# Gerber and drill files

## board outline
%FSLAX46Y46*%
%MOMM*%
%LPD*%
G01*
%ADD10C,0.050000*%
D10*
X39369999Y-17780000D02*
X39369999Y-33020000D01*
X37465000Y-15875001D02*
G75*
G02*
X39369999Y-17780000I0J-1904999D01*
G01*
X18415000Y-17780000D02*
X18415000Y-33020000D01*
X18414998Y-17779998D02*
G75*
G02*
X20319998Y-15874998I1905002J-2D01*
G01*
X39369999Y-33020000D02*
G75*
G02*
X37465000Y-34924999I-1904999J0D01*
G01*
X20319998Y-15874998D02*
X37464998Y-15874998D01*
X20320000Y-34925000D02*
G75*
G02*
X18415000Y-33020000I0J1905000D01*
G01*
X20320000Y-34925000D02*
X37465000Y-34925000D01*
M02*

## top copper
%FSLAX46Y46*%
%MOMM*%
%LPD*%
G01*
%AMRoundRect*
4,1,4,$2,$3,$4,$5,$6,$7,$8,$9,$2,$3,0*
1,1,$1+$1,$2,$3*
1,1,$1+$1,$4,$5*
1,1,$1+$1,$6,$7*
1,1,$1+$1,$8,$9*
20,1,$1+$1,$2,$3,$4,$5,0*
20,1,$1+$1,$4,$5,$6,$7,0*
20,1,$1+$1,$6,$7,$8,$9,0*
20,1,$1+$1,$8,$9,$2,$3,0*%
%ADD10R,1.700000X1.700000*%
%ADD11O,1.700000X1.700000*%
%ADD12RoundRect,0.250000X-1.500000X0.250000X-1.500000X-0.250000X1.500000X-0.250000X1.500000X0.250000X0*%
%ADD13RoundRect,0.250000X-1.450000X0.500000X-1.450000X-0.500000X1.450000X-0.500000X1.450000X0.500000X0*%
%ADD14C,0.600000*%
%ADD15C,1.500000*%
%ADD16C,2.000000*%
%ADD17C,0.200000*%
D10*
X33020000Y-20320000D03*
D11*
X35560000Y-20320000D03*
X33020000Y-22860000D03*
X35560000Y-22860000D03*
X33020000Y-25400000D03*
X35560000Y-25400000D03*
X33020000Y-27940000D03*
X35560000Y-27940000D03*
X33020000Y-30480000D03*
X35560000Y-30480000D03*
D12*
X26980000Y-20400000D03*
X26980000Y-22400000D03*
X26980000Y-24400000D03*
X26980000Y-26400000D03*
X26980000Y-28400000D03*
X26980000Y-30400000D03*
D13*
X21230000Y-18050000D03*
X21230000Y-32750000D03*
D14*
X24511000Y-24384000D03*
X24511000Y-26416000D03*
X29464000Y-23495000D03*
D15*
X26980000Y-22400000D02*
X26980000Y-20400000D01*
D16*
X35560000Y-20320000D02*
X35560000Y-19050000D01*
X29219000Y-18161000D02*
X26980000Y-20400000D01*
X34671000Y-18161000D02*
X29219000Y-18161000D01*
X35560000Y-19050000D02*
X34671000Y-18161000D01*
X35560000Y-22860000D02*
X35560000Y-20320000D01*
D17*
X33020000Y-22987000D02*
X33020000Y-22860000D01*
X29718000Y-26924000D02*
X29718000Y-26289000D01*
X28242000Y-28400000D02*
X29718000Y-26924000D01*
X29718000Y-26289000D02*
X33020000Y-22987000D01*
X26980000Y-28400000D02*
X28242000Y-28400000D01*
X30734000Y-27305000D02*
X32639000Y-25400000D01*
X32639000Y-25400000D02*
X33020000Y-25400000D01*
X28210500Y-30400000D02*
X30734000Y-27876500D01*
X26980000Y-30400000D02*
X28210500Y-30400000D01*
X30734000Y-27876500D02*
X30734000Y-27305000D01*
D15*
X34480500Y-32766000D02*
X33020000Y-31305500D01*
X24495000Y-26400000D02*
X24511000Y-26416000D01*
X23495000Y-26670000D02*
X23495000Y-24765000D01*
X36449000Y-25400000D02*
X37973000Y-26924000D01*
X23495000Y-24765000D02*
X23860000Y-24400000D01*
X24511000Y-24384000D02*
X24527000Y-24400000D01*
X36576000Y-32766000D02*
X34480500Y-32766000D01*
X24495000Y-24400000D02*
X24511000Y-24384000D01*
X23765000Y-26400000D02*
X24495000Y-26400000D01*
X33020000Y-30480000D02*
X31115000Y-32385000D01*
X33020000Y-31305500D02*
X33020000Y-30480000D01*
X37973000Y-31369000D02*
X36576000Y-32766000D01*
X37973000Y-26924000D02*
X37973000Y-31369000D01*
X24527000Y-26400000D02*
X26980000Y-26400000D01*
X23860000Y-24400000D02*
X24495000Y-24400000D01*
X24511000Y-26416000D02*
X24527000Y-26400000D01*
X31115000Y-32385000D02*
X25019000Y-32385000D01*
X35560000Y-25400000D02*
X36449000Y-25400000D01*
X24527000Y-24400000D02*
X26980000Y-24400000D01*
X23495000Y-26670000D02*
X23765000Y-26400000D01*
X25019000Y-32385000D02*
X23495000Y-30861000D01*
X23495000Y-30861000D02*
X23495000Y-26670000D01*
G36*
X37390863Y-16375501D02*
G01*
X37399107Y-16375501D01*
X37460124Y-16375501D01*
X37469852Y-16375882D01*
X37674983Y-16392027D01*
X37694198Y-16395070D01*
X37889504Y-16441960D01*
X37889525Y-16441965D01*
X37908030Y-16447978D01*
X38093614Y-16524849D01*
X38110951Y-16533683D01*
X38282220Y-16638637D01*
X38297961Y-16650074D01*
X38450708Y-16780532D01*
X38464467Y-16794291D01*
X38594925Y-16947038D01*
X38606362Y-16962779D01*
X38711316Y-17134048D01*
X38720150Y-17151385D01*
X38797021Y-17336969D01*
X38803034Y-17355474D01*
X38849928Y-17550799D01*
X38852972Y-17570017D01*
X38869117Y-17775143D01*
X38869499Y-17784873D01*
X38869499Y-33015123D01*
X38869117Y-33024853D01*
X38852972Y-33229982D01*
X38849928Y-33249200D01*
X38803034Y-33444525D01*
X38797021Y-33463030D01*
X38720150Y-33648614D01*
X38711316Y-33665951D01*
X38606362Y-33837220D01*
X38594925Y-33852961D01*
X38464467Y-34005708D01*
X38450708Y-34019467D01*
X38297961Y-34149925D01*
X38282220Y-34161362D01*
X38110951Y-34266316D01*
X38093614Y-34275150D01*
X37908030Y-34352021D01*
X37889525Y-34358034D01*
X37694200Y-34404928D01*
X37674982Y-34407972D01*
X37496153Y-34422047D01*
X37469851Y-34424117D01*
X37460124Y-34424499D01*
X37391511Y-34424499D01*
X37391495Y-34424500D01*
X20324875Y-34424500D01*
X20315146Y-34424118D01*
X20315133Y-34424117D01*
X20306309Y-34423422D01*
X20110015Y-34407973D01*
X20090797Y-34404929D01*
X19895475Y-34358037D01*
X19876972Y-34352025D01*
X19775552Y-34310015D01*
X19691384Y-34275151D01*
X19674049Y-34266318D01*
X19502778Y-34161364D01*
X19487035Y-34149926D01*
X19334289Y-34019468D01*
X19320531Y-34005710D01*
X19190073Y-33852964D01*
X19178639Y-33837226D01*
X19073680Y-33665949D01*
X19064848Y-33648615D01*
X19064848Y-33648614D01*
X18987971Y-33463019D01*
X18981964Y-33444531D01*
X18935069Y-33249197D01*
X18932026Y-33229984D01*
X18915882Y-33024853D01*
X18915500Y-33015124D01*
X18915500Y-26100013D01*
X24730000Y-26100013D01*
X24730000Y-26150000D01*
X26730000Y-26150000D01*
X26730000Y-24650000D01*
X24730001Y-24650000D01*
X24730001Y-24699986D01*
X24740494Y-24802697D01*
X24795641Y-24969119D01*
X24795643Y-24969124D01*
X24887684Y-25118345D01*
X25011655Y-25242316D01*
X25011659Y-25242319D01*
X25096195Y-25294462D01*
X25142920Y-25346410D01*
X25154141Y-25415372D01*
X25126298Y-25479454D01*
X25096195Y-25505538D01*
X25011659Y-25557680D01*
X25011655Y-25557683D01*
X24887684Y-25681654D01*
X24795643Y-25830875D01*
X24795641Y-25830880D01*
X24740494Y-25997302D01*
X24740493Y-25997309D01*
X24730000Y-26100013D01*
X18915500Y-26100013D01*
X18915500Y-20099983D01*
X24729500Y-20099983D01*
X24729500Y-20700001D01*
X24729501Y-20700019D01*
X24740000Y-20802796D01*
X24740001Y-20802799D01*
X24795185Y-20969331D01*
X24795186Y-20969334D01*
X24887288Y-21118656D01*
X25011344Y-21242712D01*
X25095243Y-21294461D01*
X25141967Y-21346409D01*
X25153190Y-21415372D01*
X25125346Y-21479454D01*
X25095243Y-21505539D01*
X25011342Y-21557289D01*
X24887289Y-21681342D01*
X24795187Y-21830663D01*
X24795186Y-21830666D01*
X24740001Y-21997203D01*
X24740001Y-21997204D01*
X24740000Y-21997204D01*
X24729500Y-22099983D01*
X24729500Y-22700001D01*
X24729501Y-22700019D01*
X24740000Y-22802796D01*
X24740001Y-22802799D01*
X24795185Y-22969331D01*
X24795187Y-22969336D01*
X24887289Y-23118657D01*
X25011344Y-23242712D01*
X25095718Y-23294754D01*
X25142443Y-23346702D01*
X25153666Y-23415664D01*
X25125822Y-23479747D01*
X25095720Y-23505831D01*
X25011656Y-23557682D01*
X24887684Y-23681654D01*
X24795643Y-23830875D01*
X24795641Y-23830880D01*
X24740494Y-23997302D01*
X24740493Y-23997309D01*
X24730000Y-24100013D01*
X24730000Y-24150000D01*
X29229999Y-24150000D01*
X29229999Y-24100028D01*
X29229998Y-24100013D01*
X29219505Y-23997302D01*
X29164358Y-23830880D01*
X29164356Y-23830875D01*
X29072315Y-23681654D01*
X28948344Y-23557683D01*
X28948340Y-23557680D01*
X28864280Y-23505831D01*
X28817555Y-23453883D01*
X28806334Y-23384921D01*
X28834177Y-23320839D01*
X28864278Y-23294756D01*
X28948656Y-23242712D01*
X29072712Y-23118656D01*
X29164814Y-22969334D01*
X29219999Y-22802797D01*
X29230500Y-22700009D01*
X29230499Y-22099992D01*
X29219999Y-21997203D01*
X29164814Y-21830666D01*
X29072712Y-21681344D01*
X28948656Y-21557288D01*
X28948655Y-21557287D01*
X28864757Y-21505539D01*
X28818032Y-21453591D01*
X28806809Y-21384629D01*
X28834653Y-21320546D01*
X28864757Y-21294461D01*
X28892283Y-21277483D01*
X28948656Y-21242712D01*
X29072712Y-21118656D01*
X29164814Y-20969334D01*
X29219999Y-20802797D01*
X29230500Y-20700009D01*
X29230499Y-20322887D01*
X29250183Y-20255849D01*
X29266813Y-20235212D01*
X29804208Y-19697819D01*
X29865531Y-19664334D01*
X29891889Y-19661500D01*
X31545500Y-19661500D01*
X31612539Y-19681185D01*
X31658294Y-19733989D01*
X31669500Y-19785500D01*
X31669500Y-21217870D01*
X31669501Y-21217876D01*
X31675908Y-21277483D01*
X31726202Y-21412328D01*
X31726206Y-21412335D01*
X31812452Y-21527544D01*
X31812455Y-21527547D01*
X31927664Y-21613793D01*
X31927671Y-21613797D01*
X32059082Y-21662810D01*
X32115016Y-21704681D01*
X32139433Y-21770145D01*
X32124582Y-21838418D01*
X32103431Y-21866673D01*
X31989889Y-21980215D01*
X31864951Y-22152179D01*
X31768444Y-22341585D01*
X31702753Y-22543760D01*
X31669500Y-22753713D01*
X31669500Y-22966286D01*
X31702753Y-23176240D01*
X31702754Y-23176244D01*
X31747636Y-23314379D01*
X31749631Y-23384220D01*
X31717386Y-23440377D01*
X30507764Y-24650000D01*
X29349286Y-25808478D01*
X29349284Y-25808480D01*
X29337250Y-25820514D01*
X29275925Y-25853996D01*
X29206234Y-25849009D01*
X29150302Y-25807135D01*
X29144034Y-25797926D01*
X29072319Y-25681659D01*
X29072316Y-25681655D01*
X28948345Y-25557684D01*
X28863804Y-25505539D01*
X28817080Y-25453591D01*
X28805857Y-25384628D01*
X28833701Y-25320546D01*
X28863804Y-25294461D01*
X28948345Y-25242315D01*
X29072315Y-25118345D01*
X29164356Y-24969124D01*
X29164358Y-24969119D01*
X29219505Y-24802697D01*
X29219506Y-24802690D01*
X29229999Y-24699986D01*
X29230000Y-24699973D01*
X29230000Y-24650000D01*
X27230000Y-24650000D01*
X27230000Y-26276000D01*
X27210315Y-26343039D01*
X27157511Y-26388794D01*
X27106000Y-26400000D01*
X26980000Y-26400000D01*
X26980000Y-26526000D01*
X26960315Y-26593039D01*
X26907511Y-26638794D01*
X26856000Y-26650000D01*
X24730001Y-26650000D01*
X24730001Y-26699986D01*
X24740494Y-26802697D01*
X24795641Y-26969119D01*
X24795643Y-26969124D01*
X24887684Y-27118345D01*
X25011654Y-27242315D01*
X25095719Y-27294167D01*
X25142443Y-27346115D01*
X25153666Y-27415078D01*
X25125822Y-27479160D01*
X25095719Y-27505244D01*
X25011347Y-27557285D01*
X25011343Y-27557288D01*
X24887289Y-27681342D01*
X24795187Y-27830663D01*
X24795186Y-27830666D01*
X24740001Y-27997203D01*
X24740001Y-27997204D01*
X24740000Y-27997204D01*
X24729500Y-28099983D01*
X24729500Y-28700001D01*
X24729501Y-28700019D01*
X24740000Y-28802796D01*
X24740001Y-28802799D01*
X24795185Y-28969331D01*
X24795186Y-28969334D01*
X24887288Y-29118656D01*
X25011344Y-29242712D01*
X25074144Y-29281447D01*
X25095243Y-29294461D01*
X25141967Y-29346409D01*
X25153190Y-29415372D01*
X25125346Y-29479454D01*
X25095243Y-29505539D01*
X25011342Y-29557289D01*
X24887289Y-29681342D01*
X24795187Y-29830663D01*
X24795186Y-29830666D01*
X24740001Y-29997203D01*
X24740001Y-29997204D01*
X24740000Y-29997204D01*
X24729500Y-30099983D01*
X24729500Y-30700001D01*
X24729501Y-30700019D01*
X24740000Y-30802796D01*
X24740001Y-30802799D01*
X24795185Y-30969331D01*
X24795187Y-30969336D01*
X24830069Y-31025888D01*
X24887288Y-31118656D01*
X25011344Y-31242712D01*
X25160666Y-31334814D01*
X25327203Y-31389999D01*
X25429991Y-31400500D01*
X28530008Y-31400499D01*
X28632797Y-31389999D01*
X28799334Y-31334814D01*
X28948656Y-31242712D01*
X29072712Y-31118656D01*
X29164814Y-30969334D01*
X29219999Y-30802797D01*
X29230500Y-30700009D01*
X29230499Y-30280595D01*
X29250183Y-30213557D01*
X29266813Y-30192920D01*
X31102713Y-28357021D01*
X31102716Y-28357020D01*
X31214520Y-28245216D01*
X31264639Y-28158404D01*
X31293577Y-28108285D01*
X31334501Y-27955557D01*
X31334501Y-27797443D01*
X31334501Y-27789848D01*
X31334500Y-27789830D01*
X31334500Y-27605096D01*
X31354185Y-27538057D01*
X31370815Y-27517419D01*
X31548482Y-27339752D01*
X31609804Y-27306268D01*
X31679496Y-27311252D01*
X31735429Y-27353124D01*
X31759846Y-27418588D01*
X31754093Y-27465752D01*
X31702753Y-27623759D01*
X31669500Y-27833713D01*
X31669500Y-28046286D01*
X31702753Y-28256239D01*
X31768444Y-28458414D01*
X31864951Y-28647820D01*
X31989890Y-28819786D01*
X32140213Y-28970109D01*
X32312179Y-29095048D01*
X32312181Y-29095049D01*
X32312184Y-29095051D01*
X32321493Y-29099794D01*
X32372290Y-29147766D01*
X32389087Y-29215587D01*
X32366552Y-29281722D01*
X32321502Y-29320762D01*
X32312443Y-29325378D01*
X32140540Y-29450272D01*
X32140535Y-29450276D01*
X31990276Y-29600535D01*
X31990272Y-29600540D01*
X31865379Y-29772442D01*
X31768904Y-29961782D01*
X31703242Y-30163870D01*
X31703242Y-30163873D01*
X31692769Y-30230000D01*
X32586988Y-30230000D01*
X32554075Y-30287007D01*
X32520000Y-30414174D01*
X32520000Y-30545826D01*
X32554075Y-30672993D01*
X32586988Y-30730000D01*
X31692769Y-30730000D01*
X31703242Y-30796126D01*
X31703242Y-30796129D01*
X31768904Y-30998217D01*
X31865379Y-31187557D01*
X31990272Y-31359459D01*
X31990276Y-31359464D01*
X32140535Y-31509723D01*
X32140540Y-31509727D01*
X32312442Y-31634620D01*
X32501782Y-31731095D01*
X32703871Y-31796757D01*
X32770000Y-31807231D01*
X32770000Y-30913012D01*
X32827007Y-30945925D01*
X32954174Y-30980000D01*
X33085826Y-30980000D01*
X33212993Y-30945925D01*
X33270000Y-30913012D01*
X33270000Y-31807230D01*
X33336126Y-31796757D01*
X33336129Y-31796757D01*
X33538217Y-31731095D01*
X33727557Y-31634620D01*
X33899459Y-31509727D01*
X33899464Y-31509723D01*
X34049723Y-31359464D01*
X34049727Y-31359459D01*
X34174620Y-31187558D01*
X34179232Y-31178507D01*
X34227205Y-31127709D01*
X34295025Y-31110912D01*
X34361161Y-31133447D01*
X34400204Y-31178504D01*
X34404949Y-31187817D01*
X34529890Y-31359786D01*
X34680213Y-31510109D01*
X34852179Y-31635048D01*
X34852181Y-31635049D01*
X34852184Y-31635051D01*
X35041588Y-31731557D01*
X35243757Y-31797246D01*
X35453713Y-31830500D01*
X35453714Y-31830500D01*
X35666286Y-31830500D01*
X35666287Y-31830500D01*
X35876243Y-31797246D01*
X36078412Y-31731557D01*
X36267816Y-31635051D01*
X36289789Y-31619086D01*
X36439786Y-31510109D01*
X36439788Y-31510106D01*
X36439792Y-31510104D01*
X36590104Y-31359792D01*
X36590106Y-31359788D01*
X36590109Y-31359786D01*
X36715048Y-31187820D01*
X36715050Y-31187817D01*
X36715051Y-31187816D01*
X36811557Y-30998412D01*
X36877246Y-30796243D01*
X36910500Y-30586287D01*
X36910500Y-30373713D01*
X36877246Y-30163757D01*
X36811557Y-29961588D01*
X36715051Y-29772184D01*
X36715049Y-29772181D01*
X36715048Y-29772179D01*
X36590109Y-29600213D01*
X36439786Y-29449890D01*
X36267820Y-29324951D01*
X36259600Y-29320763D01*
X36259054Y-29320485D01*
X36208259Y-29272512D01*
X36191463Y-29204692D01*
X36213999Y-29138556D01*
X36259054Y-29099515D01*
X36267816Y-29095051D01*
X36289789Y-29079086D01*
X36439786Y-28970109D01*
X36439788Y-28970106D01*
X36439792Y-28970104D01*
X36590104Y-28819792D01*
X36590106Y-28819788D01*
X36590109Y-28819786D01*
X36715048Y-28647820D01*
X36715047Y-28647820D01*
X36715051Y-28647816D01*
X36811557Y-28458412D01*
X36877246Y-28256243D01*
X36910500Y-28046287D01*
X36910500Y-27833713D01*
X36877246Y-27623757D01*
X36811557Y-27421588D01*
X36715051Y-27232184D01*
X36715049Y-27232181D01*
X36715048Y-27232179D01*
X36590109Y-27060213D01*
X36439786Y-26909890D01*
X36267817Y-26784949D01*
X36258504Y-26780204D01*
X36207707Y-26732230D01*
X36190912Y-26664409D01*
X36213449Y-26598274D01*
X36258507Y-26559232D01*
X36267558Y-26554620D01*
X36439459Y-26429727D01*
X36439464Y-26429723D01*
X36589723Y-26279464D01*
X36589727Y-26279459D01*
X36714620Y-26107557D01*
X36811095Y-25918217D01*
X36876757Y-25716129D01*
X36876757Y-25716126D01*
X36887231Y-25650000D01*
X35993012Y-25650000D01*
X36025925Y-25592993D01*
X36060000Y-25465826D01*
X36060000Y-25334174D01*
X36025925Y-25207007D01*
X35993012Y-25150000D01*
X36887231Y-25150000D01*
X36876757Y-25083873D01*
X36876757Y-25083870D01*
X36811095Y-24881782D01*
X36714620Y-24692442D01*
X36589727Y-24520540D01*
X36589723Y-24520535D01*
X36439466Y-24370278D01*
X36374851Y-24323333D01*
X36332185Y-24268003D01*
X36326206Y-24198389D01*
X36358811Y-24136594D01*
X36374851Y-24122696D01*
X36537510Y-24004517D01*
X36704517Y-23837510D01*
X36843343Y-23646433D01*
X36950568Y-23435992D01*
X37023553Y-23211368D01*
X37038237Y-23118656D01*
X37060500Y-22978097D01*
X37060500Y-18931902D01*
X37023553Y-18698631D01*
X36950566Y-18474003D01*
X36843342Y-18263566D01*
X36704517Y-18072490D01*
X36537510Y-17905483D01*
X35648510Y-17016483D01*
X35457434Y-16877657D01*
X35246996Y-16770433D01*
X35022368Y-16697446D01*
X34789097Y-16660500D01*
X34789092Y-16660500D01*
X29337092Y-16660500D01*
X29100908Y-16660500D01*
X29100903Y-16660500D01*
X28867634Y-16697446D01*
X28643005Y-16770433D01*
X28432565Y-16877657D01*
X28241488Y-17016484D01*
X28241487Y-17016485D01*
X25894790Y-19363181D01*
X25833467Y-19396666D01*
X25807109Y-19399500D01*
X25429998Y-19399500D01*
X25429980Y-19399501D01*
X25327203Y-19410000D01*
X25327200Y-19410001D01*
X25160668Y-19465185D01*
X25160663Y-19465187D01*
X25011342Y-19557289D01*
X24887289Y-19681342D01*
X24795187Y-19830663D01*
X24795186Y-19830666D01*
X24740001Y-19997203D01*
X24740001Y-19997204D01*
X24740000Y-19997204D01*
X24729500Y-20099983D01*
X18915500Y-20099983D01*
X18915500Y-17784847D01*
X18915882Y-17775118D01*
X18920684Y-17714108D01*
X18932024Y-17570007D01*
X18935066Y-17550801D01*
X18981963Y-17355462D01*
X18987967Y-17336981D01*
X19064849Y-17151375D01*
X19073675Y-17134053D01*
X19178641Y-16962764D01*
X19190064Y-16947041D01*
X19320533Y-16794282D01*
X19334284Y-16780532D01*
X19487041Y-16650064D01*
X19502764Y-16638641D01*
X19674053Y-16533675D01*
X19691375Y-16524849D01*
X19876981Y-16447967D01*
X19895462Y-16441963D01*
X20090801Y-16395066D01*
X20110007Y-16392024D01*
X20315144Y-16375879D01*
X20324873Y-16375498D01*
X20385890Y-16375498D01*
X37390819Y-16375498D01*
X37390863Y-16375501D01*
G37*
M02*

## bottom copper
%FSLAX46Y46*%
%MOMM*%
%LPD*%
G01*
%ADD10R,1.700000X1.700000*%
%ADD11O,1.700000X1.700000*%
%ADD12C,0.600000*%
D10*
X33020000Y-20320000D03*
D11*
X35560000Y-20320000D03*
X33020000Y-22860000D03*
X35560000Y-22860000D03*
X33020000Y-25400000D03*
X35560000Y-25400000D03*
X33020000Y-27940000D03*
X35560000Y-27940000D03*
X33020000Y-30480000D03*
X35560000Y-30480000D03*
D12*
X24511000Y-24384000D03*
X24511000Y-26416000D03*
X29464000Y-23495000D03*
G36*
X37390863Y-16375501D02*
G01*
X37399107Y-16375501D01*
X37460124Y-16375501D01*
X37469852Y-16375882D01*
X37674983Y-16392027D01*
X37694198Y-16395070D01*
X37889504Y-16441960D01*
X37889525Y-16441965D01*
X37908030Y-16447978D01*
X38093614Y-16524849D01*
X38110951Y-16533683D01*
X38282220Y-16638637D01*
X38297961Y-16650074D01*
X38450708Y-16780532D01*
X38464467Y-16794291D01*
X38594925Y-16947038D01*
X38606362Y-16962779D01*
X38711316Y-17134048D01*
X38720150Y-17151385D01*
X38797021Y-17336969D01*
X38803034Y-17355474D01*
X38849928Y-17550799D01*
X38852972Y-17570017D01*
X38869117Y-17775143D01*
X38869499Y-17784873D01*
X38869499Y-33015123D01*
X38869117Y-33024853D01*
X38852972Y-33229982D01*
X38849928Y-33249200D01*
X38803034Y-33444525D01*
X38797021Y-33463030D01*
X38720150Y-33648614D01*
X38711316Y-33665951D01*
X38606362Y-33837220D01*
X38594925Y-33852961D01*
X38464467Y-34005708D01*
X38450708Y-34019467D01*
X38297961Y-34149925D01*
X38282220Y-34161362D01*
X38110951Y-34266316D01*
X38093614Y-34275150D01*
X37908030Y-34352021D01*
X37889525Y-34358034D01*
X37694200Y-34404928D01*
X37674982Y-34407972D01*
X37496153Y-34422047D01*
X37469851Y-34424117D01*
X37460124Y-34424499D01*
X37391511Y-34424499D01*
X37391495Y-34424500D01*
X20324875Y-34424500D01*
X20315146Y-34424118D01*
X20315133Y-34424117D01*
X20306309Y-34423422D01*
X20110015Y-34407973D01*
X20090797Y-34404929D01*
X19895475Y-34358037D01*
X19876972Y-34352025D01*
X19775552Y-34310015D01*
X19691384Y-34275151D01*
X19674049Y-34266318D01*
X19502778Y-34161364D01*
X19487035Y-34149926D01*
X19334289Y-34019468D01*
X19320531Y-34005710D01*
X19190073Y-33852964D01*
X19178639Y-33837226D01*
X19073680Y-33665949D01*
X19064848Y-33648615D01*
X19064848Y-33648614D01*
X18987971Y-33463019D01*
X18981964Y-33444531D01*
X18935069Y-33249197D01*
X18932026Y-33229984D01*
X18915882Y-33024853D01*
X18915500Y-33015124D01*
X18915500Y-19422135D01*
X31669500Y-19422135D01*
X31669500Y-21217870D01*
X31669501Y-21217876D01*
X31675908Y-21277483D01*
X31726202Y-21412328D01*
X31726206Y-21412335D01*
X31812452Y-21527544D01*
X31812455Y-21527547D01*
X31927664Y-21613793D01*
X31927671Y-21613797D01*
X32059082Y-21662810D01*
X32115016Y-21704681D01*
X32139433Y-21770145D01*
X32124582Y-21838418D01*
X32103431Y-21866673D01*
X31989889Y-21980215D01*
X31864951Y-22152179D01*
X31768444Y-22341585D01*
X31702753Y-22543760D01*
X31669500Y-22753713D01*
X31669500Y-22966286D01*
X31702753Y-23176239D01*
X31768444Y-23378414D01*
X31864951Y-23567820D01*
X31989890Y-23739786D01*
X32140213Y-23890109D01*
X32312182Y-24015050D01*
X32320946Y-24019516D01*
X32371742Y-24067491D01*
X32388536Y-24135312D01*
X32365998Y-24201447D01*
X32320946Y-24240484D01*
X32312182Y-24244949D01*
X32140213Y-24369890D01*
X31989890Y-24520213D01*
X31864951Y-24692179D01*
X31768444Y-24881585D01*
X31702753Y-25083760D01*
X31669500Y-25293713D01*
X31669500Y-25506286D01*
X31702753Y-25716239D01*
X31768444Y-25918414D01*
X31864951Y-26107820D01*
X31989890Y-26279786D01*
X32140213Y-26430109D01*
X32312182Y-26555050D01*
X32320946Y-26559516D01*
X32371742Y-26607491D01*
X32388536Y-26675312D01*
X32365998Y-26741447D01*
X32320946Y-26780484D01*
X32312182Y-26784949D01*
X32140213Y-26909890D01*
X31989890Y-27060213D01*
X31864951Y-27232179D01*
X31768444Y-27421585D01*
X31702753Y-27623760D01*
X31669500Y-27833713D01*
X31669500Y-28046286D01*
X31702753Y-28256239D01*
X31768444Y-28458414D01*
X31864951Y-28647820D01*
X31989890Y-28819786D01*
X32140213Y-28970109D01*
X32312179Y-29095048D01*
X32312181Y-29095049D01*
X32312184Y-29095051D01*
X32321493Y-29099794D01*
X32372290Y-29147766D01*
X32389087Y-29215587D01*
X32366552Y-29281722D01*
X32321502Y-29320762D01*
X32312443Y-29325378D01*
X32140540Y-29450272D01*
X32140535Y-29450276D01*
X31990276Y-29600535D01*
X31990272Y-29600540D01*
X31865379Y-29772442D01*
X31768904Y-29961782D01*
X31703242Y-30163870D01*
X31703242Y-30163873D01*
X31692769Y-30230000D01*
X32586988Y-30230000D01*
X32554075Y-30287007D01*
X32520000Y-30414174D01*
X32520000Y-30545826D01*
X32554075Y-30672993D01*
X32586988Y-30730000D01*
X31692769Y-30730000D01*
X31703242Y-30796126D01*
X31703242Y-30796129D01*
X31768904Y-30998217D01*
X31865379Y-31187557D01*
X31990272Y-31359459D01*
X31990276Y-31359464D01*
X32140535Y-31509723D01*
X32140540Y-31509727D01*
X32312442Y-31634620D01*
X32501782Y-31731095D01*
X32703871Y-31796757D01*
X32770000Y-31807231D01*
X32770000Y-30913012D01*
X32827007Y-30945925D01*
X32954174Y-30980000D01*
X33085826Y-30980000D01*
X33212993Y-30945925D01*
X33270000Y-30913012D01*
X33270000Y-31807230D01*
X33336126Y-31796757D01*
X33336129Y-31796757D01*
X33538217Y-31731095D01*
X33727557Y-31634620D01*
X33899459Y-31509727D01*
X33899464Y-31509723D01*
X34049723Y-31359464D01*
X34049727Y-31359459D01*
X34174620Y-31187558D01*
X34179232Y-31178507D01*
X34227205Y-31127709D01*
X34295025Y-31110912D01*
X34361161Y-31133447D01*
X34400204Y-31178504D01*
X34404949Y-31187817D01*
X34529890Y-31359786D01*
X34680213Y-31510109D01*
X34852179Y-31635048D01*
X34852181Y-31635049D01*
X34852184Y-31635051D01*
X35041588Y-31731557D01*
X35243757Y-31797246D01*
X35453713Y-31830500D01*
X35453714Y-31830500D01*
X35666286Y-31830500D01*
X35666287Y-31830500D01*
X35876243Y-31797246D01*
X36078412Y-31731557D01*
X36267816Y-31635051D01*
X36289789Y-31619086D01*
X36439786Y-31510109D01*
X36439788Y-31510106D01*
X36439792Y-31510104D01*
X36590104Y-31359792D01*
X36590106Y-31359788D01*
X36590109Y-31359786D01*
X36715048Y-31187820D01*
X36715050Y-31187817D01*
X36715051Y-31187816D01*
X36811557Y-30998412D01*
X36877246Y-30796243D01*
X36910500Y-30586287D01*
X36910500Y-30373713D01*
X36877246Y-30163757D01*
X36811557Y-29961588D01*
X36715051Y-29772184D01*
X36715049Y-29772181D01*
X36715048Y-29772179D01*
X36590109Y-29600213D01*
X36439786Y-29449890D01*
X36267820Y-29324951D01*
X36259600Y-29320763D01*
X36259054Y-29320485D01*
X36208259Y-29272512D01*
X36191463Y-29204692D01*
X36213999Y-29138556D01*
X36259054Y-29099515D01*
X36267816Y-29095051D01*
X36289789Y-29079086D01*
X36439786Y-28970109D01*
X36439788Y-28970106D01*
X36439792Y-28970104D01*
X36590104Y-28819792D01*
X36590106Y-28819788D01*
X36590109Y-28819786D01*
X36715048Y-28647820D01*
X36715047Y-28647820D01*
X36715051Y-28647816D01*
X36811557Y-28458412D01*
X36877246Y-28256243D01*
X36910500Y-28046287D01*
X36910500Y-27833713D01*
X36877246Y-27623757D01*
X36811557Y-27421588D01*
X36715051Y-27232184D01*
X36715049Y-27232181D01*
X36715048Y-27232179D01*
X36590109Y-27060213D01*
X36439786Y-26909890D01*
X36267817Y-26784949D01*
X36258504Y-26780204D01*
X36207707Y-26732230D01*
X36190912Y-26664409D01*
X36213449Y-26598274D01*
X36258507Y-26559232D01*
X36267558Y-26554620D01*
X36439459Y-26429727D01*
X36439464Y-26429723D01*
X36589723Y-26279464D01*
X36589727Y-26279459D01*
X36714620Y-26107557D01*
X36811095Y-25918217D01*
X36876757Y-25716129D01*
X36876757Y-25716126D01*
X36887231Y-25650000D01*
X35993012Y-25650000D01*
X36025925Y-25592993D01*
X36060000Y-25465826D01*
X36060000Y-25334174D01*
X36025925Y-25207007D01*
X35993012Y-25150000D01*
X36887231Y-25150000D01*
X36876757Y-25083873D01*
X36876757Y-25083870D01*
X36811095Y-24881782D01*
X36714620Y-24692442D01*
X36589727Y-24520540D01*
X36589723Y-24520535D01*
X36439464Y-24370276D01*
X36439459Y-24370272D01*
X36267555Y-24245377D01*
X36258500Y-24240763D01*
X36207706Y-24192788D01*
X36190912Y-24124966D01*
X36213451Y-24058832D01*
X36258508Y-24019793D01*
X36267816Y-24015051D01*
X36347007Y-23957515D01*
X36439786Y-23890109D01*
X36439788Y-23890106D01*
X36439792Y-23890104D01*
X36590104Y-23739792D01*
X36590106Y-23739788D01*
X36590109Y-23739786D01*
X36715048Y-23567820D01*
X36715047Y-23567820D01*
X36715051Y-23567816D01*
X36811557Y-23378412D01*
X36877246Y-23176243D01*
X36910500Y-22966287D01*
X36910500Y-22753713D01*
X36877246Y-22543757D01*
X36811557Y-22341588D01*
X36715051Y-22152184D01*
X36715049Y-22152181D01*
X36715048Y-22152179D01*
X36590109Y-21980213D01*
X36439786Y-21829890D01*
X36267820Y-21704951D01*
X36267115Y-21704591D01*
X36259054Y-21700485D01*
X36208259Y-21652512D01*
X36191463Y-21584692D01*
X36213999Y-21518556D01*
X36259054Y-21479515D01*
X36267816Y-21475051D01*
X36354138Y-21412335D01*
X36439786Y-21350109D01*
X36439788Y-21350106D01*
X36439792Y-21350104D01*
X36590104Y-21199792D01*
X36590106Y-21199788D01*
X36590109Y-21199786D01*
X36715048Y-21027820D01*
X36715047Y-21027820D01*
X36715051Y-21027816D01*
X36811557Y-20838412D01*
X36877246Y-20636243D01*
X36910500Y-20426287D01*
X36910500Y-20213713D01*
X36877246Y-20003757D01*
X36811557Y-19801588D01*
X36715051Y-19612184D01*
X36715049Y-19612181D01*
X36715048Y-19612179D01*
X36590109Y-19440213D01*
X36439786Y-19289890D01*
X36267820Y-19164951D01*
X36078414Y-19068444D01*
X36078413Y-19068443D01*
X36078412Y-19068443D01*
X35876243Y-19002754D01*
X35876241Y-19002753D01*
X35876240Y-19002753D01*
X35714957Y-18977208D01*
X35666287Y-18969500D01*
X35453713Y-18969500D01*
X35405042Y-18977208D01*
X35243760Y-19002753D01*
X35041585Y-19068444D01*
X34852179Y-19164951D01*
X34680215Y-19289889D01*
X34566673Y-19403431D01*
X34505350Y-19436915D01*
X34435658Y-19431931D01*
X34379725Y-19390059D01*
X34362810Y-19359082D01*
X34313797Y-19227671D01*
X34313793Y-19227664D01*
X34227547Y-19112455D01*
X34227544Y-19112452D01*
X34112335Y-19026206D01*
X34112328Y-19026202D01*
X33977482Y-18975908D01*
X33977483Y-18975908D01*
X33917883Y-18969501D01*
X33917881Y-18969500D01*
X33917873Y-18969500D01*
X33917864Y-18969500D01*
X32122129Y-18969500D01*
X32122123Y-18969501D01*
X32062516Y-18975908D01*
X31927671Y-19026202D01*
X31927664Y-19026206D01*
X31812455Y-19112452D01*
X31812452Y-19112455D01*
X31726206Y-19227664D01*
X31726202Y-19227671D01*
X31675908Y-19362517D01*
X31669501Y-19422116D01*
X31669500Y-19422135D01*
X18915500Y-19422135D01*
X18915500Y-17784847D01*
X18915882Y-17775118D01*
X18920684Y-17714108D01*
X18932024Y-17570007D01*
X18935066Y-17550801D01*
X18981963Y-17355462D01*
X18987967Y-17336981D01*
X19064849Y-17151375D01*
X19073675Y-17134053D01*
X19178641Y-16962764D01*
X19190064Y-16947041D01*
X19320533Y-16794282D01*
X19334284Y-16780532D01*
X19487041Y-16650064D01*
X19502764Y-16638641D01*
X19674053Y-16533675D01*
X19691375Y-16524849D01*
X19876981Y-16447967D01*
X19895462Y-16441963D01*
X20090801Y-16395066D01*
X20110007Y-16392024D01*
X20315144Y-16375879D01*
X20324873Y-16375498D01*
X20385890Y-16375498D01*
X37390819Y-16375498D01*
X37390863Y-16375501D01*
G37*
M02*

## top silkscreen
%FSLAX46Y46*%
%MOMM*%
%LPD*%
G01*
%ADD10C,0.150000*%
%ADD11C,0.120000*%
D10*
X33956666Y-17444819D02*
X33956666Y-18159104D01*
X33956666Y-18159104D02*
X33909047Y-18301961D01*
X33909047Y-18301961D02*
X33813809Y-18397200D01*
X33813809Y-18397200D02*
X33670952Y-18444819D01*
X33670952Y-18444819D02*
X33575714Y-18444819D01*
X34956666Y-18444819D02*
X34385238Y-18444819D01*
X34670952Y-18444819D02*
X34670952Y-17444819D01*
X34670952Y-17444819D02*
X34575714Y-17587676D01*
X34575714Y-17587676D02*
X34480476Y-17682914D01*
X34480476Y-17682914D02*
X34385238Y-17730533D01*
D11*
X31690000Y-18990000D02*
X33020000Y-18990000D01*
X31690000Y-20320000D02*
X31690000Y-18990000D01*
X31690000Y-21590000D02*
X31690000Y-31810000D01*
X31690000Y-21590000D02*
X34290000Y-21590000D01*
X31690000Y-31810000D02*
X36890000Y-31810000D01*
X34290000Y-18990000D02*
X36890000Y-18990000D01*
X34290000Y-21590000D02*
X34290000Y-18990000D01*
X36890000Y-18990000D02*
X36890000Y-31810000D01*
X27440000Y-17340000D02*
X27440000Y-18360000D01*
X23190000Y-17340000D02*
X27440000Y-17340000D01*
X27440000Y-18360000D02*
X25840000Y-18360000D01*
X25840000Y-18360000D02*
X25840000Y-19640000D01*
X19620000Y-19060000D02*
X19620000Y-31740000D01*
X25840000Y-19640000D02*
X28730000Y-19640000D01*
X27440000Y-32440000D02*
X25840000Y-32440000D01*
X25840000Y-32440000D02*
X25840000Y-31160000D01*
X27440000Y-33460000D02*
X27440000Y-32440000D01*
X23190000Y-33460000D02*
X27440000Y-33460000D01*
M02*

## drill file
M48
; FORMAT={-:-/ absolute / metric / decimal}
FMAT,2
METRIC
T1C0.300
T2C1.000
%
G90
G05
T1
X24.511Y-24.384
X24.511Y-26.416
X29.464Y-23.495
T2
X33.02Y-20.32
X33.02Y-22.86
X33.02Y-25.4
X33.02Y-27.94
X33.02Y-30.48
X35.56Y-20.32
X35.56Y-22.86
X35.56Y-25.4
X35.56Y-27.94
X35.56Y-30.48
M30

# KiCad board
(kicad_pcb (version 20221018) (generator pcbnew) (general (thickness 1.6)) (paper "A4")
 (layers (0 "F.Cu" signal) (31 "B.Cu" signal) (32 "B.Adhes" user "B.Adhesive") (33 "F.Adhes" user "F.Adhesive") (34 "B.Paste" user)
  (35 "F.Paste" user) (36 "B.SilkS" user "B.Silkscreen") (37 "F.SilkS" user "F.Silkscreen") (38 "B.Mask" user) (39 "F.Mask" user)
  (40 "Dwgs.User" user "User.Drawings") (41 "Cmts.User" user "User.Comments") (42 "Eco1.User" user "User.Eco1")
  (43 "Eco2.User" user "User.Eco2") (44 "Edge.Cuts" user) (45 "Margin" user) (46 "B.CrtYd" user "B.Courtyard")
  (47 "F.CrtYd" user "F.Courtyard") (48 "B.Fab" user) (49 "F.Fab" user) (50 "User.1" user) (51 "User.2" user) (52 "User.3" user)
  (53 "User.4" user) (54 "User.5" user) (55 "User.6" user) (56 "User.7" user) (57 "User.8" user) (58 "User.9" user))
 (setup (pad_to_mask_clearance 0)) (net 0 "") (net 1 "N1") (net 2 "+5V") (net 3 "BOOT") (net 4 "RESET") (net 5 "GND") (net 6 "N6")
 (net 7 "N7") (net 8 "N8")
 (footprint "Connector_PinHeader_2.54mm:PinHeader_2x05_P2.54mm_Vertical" (layer "F.Cu") (at 33.02 20.32)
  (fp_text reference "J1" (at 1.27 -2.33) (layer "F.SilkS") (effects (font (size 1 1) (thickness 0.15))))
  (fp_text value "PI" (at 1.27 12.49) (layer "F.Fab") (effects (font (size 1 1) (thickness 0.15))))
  (fp_line (start -1.33 -1.33) (end 0 -1.33) (stroke (width 0.12) (type solid)) (layer "F.SilkS"))
  (fp_line (start -1.33 0) (end -1.33 -1.33) (stroke (width 0.12) (type solid)) (layer "F.SilkS"))
  (fp_line (start -1.33 1.27) (end -1.33 11.49) (stroke (width 0.12) (type solid)) (layer "F.SilkS"))
  (fp_line (start -1.33 1.27) (end 1.27 1.27) (stroke (width 0.12) (type solid)) (layer "F.SilkS"))
  (fp_line (start -1.33 11.49) (end 3.87 11.49) (stroke (width 0.12) (type solid)) (layer "F.SilkS"))
  (fp_line (start 1.27 -1.33) (end 3.87 -1.33) (stroke (width 0.12) (type solid)) (layer "F.SilkS"))
  (fp_line (start 1.27 1.27) (end 1.27 -1.33) (stroke (width 0.12) (type solid)) (layer "F.SilkS"))
  (fp_line (start 3.87 -1.33) (end 3.87 11.49) (stroke (width 0.12) (type solid)) (layer "F.SilkS"))
  (pad "1" thru_hole rect (at 0 0) (size 1.7 1.7) (drill 1) (layers "*.Cu" "*.Mask") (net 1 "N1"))
  (pad "2" thru_hole oval (at 2.54 0) (size 1.7 1.7) (drill 1) (layers "*.Cu" "*.Mask") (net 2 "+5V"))
  (pad "3" thru_hole oval (at 0 2.54) (size 1.7 1.7) (drill 1) (layers "*.Cu" "*.Mask") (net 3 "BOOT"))
  (pad "4" thru_hole oval (at 2.54 2.54) (size 1.7 1.7) (drill 1) (layers "*.Cu" "*.Mask") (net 2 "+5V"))
  (pad "5" thru_hole oval (at 0 5.08) (size 1.7 1.7) (drill 1) (layers "*.Cu" "*.Mask") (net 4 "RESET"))
  (pad "6" thru_hole oval (at 2.54 5.08) (size 1.7 1.7) (drill 1) (layers "*.Cu" "*.Mask") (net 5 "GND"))
  (pad "7" thru_hole oval (at 0 7.62) (size 1.7 1.7) (drill 1) (layers "*.Cu" "*.Mask") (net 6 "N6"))
  (pad "8" thru_hole oval (at 2.54 7.62) (size 1.7 1.7) (drill 1) (layers "*.Cu" "*.Mask") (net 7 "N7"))
  (pad "9" thru_hole oval (at 0 10.16) (size 1.7 1.7) (drill 1) (layers "*.Cu" "*.Mask") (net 5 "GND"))
  (pad "10" thru_hole oval (at 2.54 10.16) (size 1.7 1.7) (drill 1) (layers "*.Cu" "*.Mask") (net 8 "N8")))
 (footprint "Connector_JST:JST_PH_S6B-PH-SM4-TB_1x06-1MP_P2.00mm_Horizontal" (layer "F.Cu") (at 24.13 25.4 -90)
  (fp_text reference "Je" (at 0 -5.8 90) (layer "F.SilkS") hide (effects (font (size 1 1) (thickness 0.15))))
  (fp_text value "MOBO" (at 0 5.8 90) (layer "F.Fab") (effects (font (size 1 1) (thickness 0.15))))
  (fp_line (start -8.06 -3.31) (end -7.04 -3.31) (stroke (width 0.12) (type solid)) (layer "F.SilkS"))
  (fp_line (start -8.06 0.94) (end -8.06 -3.31) (stroke (width 0.12) (type solid)) (layer "F.SilkS"))
  (fp_line (start -7.04 -3.31) (end -7.04 -1.71) (stroke (width 0.12) (type solid)) (layer "F.SilkS"))
  (fp_line (start -7.04 -1.71) (end -5.76 -1.71) (stroke (width 0.12) (type solid)) (layer "F.SilkS"))
  (fp_line (start -6.34 4.51) (end 6.34 4.51) (stroke (width 0.12) (type solid)) (layer "F.SilkS"))
  (fp_line (start -5.76 -1.71) (end -5.76 -4.6) (stroke (width 0.12) (type solid)) (layer "F.SilkS"))
  (fp_line (start 7.04 -3.31) (end 7.04 -1.71) (stroke (width 0.12) (type solid)) (layer "F.SilkS"))
  (fp_line (start 7.04 -1.71) (end 5.76 -1.71) (stroke (width 0.12) (type solid)) (layer "F.SilkS"))
  (fp_line (start 8.06 -3.31) (end 7.04 -3.31) (stroke (width 0.12) (type solid)) (layer "F.SilkS"))
  (fp_line (start 8.06 0.94) (end 8.06 -3.31) (stroke (width 0.12) (type solid)) (layer "F.SilkS"))
  (pad "1" smd roundrect (at -5 -2.85 270) (size 1 3.5) (layers "F.Cu" "F.Paste" "F.Mask") (roundrect_rratio 0.25) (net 2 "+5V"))
  (pad "2" smd roundrect (at -3 -2.85 270) (size 1 3.5) (layers "F.Cu" "F.Paste" "F.Mask") (roundrect_rratio 0.25) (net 2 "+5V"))
  (pad "3" smd roundrect (at -1 -2.85 270) (size 1 3.5) (layers "F.Cu" "F.Paste" "F.Mask") (roundrect_rratio 0.25) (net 5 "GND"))
  (pad "4" smd roundrect (at 1 -2.85 270) (size 1 3.5) (layers "F.Cu" "F.Paste" "F.Mask") (roundrect_rratio 0.25) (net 5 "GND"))
  (pad "5" smd roundrect (at 3 -2.85 270) (size 1 3.5) (layers "F.Cu" "F.Paste" "F.Mask") (roundrect_rratio 0.25) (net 3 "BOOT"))
  (pad "6" smd roundrect (at 5 -2.85 270) (size 1 3.5) (layers "F.Cu" "F.Paste" "F.Mask") (roundrect_rratio 0.25) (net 4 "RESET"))
  (pad "MP" smd roundrect (at -7.35 2.9 270) (size 1.5 3.4) (layers "F.Cu" "F.Paste" "F.Mask") (roundrect_rratio 0.1666666667) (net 5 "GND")
   (zone_connect 2))
  (pad "MP" smd roundrect (at 7.35 2.9 270) (size 1.5 3.4) (layers "F.Cu" "F.Paste" "F.Mask") (roundrect_rratio 0.1666666667) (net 5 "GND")
   (zone_connect 2)))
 (gr_line (start 39.369999 17.78) (end 39.369999 33.02) (stroke (width 0.05) (type default)) (layer "Edge.Cuts"))
 (gr_arc (start 37.465 15.875001) (mid 38.812037 16.432963) (end 39.369999 17.78) (stroke (width 0.05) (type default)) (layer "Edge.Cuts"))
 (gr_line (start 18.415 17.78) (end 18.415 33.02) (stroke (width 0.05) (type default)) (layer "Edge.Cuts"))
 (gr_arc (start 18.414998 17.779998) (mid 18.97296 16.43296) (end 20.319998 15.874998) (stroke (width 0.05) (type default))
  (layer "Edge.Cuts"))
 (gr_arc (start 39.369999 33.02) (mid 38.812037 34.367037) (end 37.465 34.924999) (stroke (width 0.05) (type default)) (layer "Edge.Cuts"))
 (gr_line (start 20.319998 15.874998) (end 37.464998 15.874998) (stroke (width 0.05) (type default)) (layer "Edge.Cuts"))
 (gr_arc (start 20.32 34.925) (mid 18.972962 34.367038) (end 18.415 33.02) (stroke (width 0.05) (type default)) (layer "Edge.Cuts"))
 (gr_line (start 20.32 34.925) (end 37.465 34.925) (stroke (width 0.05) (type default)) (layer "Edge.Cuts"))
 (segment (start 26.98 22.4) (end 26.98 20.4) (width 1.5) (layer "F.Cu") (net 2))
 (segment (start 35.56 20.32) (end 35.56 19.05) (width 2) (layer "F.Cu") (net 2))
 (segment (start 29.219 18.161) (end 26.98 20.4) (width 2) (layer "F.Cu") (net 2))
 (segment (start 34.671 18.161) (end 29.219 18.161) (width 2) (layer "F.Cu") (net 2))
 (segment (start 35.56 19.05) (end 34.671 18.161) (width 2) (layer "F.Cu") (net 2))
 (segment (start 35.56 22.86) (end 35.56 20.32) (width 2) (layer "F.Cu") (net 2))
 (segment (start 33.02 22.987) (end 33.02 22.86) (width 0.2) (layer "F.Cu") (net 3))
 (segment (start 29.718 26.924) (end 29.718 26.289) (width 0.2) (layer "F.Cu") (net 3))
 (segment (start 28.242 28.4) (end 29.718 26.924) (width 0.2) (layer "F.Cu") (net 3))
 (segment (start 29.718 26.289) (end 33.02 22.987) (width 0.2) (layer "F.Cu") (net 3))
 (segment (start 26.98 28.4) (end 28.242 28.4) (width 0.2) (layer "F.Cu") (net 3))
 (segment (start 30.734 27.305) (end 32.639 25.4) (width 0.2) (layer "F.Cu") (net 4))
 (segment (start 32.639 25.4) (end 33.02 25.4) (width 0.2) (layer "F.Cu") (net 4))
 (segment (start 28.2105 30.4) (end 30.734 27.8765) (width 0.2) (layer "F.Cu") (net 4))
 (segment (start 26.98 30.4) (end 28.2105 30.4) (width 0.2) (layer "F.Cu") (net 4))
 (segment (start 30.734 27.8765) (end 30.734 27.305) (width 0.2) (layer "F.Cu") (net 4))
 (segment (start 34.4805 32.766) (end 33.02 31.3055) (width 1.5) (layer "F.Cu") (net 5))
 (segment (start 24.495 26.4) (end 24.511 26.416) (width 1.5) (layer "F.Cu") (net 5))
 (segment (start 23.495 26.67) (end 23.495 24.765) (width 1.5) (layer "F.Cu") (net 5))
 (segment (start 36.449 25.4) (end 37.973 26.924) (width 1.5) (layer "F.Cu") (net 5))
 (segment (start 23.495 24.765) (end 23.86 24.4) (width 1.5) (layer "F.Cu") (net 5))
 (segment (start 24.511 24.384) (end 24.527 24.4) (width 1.5) (layer "F.Cu") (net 5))
 (segment (start 36.576 32.766) (end 34.4805 32.766) (width 1.5) (layer "F.Cu") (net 5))
 (segment (start 24.495 24.4) (end 24.511 24.384) (width 1.5) (layer "F.Cu") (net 5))
 (segment (start 23.765 26.4) (end 24.495 26.4) (width 1.5) (layer "F.Cu") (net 5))
 (segment (start 33.02 30.48) (end 31.115 32.385) (width 1.5) (layer "F.Cu") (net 5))
 (segment (start 33.02 31.3055) (end 33.02 30.48) (width 1.5) (layer "F.Cu") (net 5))
 (segment (start 37.973 31.369) (end 36.576 32.766) (width 1.5) (layer "F.Cu") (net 5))
 (segment (start 37.973 26.924) (end 37.973 31.369) (width 1.5) (layer "F.Cu") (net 5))
 (segment (start 24.527 26.4) (end 26.98 26.4) (width 1.5) (layer "F.Cu") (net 5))
 (segment (start 23.86 24.4) (end 24.495 24.4) (width 1.5) (layer "F.Cu") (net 5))
 (segment (start 24.511 26.416) (end 24.527 26.4) (width 1.5) (layer "F.Cu") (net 5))
 (segment (start 31.115 32.385) (end 25.019 32.385) (width 1.5) (layer "F.Cu") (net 5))
 (segment (start 35.56 25.4) (end 36.449 25.4) (width 1.5) (layer "F.Cu") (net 5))
 (segment (start 24.527 24.4) (end 26.98 24.4) (width 1.5) (layer "F.Cu") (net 5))
 (segment (start 23.495 26.67) (end 23.765 26.4) (width 1.5) (layer "F.Cu") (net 5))
 (segment (start 25.019 32.385) (end 23.495 30.861) (width 1.5) (layer "F.Cu") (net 5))
 (segment (start 23.495 30.861) (end 23.495 26.67) (width 1.5) (layer "F.Cu") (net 5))
 (via (at 24.511 24.384) (size 0.6) (drill 0.3) (layers "F.Cu" "B.Cu") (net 5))
 (via (at 24.511 26.416) (size 0.6) (drill 0.3) (layers "F.Cu" "B.Cu") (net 5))
 (via (at 29.464 23.495) (size 0.6) (drill 0.3) (layers "F.Cu" "B.Cu") (free) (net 5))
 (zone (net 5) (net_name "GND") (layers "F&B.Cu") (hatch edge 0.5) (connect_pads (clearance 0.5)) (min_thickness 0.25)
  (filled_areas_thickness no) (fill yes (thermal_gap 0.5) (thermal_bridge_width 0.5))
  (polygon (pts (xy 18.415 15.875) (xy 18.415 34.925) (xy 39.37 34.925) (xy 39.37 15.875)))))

